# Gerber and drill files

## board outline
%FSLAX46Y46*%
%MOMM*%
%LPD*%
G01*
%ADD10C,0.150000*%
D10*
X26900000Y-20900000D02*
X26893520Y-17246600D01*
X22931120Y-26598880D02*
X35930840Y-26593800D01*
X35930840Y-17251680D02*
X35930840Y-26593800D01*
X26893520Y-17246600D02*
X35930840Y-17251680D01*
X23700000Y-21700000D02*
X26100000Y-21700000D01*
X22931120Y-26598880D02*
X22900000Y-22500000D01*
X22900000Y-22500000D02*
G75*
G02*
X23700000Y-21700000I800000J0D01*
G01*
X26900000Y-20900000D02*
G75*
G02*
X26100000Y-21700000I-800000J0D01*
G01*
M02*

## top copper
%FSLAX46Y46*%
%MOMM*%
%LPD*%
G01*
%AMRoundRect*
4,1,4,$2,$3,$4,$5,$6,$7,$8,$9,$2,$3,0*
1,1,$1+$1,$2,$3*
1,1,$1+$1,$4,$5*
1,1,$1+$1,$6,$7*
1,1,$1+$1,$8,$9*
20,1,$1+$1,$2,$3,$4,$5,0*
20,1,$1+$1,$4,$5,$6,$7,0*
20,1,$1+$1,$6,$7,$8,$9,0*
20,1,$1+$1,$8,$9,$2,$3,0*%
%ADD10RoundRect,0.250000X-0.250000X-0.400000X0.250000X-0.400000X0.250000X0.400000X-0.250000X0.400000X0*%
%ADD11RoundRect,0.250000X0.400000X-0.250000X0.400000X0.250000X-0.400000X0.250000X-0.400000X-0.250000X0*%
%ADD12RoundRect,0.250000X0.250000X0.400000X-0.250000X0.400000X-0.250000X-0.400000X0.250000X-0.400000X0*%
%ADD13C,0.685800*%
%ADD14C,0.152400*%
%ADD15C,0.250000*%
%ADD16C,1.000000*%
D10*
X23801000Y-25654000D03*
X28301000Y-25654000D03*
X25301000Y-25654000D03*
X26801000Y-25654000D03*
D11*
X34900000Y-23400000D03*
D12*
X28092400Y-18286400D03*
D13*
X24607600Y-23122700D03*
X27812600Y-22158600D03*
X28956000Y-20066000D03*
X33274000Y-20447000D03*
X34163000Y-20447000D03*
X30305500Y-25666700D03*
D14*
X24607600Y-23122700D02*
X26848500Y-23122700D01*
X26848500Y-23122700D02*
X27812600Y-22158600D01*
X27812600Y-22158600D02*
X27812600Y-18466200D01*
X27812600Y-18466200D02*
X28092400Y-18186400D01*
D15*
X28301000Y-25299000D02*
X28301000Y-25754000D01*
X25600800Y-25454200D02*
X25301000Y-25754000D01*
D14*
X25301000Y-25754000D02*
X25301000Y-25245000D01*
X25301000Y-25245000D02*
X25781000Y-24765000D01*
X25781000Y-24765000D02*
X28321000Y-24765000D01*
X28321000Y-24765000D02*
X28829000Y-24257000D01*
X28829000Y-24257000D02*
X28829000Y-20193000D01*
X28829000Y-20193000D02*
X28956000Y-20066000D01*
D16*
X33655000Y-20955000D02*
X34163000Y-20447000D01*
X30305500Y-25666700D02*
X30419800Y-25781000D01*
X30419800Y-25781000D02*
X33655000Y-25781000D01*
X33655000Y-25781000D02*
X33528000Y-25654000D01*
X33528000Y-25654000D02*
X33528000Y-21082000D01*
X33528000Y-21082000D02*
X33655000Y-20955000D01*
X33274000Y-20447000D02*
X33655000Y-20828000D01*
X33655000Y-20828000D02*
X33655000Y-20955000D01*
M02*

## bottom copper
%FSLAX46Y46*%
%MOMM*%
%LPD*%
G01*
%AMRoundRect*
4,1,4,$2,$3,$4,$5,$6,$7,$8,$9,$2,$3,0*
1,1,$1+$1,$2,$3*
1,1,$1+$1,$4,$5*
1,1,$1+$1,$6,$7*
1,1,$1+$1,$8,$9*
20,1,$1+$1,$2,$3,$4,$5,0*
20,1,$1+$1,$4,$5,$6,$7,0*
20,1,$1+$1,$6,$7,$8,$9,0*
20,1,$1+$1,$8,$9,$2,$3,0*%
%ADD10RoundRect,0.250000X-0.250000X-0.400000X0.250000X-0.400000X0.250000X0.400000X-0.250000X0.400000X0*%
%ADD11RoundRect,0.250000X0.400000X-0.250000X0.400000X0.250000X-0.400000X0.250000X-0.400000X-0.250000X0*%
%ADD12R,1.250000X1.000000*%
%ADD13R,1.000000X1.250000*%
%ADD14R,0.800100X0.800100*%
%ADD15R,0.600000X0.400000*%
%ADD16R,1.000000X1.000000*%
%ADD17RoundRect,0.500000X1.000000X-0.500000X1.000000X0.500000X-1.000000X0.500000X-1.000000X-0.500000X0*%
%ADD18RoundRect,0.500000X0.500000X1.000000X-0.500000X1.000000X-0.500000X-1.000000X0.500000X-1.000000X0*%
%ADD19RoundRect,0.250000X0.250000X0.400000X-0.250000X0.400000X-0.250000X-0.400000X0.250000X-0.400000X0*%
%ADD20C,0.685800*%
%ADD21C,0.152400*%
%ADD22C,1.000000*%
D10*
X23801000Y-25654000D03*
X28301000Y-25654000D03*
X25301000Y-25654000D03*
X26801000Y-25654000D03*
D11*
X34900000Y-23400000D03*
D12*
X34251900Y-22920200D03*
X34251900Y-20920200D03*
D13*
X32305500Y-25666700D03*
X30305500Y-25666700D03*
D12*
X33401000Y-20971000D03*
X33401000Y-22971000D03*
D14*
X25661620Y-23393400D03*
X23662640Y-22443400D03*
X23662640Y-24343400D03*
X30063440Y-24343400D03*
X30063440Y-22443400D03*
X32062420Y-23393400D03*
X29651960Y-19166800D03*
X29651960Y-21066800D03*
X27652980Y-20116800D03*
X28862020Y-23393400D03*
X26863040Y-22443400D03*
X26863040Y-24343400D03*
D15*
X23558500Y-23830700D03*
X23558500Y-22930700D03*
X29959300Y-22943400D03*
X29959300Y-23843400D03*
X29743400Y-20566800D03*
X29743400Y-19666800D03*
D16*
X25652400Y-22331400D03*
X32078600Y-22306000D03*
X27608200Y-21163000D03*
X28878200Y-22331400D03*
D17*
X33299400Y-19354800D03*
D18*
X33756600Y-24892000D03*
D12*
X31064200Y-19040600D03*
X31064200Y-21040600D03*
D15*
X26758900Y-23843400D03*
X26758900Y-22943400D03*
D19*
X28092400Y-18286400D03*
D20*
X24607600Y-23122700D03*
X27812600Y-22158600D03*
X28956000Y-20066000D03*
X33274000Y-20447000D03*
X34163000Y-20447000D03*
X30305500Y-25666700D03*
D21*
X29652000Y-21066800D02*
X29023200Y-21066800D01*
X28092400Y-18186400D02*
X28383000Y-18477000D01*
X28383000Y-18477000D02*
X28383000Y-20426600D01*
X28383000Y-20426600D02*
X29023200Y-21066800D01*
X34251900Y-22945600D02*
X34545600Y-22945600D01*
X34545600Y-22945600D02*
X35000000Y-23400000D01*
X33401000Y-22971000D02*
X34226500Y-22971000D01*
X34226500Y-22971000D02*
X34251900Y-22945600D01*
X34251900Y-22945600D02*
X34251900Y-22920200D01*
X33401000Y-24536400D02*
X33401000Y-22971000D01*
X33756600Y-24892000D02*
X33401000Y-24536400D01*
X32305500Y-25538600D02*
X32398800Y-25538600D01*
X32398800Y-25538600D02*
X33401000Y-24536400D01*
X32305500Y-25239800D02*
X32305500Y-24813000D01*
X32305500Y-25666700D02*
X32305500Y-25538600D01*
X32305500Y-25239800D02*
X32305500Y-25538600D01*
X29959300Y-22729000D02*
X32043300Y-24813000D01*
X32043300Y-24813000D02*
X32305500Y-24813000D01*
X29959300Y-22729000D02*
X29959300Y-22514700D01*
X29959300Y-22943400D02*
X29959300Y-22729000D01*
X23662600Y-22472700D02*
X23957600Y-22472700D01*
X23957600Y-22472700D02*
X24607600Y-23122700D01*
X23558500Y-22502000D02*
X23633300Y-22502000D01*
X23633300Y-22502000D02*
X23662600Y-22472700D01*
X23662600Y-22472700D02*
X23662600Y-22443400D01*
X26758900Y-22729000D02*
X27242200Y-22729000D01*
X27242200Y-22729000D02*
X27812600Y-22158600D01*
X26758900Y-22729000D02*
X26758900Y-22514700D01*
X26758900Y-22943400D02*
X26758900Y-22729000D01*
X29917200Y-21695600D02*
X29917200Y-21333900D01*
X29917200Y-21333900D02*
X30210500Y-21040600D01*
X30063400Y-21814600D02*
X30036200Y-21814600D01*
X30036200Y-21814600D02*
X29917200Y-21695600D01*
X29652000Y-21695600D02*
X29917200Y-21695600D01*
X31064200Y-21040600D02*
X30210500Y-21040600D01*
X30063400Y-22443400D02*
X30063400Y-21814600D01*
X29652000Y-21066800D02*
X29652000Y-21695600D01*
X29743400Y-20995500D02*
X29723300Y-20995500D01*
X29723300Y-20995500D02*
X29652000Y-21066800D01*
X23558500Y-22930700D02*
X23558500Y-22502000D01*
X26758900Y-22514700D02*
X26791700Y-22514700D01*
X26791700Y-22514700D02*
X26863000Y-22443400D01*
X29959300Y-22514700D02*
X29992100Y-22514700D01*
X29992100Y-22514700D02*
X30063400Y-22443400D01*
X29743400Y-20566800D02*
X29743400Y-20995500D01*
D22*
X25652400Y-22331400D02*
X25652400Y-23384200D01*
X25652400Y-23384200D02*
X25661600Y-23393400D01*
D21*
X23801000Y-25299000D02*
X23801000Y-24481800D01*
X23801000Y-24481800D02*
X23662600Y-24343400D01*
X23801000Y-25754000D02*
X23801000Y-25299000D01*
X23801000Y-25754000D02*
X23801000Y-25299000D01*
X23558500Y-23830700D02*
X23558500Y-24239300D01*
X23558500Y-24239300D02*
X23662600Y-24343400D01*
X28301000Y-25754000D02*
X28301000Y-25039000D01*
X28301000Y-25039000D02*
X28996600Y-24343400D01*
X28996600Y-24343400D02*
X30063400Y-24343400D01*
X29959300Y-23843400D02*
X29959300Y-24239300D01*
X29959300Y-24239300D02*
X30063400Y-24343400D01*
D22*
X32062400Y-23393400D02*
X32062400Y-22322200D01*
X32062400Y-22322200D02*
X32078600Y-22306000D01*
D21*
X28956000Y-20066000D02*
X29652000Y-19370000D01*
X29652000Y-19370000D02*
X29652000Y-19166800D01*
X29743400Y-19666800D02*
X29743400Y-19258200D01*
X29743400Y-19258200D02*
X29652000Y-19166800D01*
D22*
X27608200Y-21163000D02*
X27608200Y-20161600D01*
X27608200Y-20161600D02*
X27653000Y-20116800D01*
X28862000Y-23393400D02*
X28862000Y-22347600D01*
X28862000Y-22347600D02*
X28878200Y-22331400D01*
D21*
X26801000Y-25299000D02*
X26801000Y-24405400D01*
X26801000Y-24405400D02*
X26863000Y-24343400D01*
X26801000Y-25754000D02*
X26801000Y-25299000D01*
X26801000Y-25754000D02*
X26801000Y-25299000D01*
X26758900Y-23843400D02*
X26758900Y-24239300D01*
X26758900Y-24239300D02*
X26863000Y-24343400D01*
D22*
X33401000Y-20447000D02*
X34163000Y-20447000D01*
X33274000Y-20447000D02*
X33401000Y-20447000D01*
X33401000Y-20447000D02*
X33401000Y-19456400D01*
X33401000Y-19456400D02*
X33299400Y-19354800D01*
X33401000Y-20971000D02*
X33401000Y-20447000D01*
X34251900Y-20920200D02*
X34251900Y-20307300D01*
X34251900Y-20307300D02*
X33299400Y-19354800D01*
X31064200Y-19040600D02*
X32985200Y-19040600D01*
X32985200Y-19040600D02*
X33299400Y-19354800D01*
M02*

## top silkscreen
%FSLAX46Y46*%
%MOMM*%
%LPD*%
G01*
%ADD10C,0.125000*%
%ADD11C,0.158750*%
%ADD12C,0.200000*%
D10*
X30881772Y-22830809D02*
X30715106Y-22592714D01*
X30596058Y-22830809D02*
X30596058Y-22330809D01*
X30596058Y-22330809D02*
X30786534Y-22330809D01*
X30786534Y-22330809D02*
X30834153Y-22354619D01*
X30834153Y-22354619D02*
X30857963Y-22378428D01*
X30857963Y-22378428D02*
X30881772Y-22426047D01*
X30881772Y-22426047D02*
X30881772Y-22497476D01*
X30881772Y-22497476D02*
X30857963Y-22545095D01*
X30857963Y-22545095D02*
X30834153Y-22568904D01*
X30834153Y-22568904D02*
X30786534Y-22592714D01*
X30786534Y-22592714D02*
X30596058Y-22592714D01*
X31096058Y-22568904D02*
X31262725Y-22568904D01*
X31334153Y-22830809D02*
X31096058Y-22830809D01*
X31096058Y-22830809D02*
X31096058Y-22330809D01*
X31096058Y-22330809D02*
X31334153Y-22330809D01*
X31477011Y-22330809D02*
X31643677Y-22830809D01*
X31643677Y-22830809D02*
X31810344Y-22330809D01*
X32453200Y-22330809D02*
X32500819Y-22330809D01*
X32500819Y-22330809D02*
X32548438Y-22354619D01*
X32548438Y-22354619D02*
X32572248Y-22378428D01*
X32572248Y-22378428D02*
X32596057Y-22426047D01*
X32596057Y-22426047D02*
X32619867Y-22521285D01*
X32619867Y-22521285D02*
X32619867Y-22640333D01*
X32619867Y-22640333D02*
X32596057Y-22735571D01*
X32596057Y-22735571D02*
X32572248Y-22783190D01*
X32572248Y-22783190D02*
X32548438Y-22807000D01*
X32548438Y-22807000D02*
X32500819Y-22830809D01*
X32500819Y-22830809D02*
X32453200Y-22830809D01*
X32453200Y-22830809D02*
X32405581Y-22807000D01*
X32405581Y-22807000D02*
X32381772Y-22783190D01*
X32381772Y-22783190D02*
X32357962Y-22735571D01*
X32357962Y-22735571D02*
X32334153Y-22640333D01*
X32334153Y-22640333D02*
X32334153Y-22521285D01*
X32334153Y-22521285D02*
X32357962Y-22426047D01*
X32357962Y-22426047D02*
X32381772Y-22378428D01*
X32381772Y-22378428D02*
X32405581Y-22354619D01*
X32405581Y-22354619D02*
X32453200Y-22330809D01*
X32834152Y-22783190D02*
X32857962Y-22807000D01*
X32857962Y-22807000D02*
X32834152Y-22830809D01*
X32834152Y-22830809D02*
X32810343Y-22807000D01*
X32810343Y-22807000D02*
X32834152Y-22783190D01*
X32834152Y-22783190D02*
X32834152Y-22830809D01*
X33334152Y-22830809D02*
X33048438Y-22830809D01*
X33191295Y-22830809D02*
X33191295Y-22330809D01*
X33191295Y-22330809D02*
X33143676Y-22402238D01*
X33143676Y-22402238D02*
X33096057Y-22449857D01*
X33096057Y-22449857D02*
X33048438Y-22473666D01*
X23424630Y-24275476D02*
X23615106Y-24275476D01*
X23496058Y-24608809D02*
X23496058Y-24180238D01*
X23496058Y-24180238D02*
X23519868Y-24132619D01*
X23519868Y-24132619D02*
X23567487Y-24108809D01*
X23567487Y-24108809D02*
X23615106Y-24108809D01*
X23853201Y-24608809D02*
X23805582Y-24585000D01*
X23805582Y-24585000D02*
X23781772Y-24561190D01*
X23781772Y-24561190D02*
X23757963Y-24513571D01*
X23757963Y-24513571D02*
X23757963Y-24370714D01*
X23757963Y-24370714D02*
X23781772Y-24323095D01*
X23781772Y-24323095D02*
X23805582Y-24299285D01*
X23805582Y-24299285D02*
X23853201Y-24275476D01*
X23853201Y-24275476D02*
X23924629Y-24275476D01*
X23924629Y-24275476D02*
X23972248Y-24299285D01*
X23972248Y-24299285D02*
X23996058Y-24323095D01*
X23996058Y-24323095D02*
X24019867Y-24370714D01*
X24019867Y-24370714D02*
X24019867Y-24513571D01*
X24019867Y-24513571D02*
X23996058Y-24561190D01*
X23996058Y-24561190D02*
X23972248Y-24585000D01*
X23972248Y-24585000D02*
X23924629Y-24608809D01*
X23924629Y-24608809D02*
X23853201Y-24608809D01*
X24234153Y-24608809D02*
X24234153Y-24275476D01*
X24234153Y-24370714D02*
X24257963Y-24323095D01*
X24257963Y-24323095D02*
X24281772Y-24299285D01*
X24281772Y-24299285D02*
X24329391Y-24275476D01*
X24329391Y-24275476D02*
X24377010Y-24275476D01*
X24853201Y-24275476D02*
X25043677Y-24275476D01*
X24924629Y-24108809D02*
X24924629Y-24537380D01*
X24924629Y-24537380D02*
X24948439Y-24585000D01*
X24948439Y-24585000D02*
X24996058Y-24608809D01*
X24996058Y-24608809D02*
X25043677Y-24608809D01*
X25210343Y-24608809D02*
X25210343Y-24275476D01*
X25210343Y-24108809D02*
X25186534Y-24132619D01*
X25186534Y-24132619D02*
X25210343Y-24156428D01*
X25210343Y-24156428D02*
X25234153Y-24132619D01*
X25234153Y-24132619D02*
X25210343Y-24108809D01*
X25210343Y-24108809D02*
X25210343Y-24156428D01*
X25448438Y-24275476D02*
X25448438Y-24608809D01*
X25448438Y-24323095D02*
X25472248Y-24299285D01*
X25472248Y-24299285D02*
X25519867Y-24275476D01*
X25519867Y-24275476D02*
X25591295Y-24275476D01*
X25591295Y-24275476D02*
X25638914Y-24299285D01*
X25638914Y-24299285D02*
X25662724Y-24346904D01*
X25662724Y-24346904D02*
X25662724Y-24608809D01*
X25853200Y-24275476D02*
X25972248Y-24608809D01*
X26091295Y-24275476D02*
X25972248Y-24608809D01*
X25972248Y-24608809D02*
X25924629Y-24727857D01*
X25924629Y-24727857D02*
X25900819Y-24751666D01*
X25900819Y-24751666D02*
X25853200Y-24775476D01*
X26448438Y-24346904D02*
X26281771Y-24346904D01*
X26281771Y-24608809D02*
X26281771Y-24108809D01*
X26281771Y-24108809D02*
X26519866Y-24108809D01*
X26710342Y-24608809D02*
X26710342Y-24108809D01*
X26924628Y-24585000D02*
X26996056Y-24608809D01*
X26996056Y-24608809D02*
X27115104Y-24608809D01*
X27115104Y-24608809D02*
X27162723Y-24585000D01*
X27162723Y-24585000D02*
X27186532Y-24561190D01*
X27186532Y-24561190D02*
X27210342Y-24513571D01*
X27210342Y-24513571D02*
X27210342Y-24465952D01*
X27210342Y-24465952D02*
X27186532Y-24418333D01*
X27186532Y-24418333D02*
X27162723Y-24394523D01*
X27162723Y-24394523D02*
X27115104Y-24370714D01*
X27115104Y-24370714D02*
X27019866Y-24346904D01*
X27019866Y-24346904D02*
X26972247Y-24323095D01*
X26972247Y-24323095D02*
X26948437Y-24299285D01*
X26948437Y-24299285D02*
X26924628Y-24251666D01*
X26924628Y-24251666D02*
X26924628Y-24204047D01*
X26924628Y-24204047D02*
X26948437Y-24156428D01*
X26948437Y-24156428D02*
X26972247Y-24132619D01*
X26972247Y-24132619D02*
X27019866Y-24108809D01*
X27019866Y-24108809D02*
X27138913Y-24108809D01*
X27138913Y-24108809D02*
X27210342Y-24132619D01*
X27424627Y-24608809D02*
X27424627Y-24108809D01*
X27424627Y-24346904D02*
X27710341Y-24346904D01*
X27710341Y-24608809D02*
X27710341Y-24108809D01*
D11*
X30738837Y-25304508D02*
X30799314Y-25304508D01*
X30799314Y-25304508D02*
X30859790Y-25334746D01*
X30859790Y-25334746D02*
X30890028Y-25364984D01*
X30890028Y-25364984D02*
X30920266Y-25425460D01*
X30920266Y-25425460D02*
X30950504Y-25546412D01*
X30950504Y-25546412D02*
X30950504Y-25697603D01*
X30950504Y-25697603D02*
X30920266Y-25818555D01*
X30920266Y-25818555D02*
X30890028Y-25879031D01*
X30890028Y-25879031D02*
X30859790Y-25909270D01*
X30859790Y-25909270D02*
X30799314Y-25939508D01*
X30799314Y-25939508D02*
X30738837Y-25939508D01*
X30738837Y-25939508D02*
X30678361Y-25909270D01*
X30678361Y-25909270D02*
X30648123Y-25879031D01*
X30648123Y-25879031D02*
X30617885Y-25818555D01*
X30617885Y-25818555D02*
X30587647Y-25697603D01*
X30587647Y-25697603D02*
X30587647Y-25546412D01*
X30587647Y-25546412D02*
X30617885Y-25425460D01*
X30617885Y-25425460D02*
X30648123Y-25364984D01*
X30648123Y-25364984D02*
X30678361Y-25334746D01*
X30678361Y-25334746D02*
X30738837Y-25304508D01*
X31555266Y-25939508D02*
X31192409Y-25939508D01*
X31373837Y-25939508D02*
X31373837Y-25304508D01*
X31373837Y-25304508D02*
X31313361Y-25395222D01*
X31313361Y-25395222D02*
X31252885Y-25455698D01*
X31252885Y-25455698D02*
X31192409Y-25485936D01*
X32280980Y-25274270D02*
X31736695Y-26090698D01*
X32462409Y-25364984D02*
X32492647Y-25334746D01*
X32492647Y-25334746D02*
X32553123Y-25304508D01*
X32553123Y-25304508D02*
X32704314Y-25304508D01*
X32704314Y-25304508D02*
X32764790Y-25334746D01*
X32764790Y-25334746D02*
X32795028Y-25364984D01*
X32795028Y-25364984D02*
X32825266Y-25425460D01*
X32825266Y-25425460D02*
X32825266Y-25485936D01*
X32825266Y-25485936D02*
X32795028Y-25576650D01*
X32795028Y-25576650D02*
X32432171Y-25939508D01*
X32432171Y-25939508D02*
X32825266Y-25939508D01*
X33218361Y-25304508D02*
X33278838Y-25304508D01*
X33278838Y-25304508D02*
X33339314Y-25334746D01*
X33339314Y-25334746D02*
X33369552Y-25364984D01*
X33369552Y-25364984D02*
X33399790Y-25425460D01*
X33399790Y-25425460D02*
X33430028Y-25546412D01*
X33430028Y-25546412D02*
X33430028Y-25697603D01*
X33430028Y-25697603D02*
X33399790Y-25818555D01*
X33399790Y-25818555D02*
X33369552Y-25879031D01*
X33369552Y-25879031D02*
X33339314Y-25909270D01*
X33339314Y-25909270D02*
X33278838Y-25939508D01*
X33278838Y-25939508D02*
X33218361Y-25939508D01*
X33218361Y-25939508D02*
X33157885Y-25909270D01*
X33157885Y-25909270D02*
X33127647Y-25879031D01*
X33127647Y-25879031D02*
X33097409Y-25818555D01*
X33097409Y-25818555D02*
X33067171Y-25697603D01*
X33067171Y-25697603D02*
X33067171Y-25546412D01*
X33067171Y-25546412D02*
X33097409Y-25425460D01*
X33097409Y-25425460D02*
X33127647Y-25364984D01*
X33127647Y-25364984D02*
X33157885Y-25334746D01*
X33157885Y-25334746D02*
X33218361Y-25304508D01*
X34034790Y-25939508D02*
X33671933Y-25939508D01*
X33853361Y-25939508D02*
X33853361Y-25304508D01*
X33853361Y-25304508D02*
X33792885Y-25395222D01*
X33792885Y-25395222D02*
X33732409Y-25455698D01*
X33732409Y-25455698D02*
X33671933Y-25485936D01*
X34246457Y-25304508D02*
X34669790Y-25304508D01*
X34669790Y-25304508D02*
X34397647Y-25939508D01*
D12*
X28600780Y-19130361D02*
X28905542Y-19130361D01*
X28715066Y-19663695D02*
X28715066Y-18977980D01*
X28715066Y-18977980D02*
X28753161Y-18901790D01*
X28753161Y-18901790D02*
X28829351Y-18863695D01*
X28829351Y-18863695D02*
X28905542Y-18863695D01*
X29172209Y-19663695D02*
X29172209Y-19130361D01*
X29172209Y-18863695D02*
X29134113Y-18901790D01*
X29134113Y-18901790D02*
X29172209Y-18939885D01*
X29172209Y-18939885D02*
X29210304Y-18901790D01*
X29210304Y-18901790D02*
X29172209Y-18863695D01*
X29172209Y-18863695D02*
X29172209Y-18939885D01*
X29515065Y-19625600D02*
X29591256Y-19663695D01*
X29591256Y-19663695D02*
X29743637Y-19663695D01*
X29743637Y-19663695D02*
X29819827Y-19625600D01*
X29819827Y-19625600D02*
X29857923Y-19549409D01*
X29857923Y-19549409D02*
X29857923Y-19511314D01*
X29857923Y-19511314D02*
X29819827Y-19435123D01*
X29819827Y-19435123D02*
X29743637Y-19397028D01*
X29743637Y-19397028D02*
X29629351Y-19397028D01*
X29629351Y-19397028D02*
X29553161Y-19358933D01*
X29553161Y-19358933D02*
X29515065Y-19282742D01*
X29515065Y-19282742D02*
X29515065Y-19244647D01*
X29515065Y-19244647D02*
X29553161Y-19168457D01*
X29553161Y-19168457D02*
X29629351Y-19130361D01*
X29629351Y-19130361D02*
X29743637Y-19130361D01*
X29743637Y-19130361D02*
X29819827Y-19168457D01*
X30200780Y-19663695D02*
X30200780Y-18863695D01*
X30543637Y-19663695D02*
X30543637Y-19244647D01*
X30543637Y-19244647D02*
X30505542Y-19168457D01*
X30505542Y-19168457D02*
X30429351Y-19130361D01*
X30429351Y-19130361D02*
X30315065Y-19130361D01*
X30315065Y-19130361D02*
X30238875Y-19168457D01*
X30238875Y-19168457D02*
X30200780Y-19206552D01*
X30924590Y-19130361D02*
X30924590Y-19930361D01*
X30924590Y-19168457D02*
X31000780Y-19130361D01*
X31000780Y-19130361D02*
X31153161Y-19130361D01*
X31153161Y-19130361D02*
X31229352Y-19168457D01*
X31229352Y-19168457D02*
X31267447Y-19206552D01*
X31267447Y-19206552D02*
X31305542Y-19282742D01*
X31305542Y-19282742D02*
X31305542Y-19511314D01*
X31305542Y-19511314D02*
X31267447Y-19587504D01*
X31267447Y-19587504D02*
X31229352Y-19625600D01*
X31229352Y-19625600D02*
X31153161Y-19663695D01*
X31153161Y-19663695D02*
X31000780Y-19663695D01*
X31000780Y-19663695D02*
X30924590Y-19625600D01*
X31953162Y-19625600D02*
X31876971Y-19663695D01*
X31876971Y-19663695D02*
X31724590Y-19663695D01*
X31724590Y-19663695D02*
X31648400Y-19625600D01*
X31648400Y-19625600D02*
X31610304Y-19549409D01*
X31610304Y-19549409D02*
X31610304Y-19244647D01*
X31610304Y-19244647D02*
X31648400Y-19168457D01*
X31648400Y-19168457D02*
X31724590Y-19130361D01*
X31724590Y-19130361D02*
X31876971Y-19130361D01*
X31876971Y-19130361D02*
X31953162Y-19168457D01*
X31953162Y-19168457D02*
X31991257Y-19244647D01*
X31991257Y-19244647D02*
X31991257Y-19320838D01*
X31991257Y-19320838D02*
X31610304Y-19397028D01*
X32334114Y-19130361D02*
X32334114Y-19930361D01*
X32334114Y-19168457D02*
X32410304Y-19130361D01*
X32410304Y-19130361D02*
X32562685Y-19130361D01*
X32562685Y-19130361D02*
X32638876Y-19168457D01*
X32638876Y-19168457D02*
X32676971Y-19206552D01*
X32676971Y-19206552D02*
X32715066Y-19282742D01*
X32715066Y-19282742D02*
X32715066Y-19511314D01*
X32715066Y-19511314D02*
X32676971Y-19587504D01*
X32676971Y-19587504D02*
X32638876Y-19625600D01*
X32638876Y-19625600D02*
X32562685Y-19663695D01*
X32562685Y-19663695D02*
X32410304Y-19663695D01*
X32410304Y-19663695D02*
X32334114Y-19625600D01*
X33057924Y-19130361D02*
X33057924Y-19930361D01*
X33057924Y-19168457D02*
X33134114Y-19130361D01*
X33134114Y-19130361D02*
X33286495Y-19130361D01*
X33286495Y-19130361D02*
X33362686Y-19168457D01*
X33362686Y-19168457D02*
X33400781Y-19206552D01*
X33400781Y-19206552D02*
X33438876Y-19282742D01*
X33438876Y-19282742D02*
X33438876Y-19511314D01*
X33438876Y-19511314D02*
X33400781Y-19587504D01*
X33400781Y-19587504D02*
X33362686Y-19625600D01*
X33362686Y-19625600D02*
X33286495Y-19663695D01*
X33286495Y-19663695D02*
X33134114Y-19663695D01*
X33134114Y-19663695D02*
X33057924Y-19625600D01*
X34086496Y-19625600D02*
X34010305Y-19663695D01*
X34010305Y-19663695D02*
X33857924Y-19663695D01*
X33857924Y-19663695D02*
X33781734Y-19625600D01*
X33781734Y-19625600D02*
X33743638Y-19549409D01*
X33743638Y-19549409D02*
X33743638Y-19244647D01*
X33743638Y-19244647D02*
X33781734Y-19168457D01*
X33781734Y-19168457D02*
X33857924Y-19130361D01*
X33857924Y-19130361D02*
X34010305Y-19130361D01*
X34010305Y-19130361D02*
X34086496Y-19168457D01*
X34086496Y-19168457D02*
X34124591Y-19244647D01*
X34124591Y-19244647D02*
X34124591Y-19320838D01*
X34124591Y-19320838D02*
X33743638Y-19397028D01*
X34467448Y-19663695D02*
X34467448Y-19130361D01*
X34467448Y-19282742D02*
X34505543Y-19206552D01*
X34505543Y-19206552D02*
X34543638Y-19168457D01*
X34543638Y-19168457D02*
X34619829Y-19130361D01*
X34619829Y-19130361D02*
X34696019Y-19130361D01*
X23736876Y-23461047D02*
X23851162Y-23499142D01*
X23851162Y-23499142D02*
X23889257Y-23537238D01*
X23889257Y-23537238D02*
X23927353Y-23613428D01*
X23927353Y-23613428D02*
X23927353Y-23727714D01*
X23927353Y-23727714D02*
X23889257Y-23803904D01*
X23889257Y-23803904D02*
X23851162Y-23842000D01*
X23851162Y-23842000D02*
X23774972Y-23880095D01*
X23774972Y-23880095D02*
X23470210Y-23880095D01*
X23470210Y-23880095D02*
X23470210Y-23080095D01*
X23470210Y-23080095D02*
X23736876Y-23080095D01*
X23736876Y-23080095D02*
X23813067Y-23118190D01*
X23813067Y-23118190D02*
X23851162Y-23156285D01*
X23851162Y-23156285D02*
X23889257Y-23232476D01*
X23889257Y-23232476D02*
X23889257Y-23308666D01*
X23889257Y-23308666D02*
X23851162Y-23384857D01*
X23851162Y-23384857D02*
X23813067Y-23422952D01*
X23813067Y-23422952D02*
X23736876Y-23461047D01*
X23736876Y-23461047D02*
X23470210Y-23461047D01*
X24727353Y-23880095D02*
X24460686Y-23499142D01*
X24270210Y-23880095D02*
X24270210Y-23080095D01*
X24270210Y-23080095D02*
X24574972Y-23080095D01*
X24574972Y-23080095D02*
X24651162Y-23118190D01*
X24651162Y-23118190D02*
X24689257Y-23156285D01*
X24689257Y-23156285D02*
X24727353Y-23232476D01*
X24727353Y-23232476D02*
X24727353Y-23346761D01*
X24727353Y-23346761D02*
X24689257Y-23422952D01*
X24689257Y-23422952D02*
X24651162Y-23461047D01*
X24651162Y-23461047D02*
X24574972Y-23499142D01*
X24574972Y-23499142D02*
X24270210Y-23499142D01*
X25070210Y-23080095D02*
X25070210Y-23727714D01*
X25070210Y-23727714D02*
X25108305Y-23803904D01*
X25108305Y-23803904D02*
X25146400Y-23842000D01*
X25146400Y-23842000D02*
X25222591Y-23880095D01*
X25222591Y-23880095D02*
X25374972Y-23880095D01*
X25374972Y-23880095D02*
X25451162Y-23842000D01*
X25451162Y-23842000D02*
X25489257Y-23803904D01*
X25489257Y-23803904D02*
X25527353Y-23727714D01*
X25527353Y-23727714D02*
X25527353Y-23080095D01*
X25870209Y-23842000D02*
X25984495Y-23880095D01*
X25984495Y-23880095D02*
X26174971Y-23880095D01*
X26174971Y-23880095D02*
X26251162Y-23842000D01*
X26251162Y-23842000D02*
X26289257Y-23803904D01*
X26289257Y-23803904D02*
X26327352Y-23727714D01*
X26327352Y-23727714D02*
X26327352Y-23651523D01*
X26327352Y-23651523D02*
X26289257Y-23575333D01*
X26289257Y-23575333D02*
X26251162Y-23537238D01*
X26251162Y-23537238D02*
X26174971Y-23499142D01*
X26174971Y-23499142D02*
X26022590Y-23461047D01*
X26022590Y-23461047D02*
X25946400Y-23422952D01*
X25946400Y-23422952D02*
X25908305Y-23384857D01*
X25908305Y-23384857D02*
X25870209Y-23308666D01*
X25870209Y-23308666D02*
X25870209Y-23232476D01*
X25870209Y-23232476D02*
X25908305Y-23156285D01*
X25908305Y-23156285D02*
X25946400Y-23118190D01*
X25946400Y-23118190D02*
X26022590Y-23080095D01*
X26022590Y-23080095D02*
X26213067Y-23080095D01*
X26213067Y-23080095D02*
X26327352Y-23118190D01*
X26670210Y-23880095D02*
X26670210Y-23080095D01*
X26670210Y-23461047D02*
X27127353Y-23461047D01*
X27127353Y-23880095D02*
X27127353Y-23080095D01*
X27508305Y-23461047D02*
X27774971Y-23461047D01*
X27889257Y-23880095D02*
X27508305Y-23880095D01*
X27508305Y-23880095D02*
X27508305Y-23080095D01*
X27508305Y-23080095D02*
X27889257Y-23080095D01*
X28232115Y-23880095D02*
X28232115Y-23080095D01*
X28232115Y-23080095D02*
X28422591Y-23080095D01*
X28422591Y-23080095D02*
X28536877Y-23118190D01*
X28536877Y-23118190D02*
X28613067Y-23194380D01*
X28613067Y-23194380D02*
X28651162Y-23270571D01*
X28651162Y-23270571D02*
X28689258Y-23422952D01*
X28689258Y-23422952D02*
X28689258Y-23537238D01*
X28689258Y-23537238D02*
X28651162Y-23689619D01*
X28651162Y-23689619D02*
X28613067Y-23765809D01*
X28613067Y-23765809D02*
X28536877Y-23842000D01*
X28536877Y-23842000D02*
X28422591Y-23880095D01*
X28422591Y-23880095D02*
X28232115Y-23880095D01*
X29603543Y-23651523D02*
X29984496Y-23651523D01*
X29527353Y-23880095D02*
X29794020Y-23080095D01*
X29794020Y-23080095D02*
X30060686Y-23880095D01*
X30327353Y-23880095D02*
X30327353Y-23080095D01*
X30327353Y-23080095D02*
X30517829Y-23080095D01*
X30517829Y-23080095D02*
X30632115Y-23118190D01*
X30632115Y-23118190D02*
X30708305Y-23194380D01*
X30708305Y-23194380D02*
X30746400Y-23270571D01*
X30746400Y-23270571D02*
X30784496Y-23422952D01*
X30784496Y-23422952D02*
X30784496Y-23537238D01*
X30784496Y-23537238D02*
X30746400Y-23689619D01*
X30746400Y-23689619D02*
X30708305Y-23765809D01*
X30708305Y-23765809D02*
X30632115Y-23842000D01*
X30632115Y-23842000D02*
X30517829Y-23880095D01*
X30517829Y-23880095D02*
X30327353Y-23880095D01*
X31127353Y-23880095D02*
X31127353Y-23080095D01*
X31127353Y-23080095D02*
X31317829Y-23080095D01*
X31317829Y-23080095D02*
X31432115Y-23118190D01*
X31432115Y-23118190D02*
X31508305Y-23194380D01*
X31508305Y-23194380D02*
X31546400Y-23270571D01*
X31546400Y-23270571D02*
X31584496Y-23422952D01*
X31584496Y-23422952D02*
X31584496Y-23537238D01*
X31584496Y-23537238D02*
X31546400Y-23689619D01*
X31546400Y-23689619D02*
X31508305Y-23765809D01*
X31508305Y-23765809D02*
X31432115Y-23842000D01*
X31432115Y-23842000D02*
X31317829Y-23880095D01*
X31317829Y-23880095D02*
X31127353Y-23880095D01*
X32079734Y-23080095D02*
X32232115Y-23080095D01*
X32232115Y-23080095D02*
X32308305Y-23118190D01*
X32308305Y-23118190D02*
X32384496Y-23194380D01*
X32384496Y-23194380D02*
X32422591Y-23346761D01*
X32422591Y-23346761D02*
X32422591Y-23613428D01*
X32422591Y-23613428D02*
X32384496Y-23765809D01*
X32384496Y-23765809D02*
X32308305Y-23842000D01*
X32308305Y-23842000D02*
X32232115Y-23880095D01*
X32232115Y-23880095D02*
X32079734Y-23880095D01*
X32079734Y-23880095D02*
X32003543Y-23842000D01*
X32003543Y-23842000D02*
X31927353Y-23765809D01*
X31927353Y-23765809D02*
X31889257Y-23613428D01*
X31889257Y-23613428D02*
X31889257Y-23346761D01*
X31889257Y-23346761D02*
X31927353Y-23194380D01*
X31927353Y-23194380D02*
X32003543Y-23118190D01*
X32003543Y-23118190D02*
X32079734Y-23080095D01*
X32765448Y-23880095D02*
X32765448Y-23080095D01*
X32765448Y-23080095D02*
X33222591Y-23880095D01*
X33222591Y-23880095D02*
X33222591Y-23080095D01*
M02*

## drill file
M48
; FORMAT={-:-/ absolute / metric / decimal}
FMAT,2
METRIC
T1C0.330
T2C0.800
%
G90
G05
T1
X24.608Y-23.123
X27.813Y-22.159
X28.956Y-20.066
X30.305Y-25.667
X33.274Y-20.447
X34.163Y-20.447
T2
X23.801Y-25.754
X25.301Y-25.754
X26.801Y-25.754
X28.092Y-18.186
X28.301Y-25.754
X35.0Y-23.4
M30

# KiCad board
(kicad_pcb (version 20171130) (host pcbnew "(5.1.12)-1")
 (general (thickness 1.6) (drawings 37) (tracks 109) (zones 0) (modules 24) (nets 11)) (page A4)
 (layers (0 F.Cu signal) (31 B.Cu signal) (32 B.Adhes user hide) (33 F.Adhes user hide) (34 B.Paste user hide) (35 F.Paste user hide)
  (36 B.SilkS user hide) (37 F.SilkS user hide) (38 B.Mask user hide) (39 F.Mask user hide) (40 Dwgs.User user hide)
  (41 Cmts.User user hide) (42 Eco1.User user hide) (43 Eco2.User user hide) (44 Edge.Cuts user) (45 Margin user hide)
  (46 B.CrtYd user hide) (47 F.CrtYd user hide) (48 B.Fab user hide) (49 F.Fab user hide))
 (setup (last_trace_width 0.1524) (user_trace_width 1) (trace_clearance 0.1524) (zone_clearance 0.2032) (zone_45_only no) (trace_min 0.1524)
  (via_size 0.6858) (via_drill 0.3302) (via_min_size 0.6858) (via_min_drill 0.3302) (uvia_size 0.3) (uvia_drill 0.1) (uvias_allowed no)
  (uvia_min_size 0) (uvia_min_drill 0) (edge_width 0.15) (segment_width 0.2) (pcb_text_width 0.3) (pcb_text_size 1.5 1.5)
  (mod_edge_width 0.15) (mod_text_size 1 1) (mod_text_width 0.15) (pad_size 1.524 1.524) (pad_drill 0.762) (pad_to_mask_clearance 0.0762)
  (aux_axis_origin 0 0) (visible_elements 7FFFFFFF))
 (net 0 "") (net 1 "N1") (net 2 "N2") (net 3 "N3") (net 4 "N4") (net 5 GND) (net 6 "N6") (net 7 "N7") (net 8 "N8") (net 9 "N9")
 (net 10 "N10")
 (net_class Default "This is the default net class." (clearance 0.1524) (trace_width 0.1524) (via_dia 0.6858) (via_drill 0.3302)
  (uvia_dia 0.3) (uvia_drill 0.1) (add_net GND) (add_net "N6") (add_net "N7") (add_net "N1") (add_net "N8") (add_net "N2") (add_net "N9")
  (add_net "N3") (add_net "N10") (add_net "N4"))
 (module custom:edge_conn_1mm (layer F.Cu) (at 23.801 25.754)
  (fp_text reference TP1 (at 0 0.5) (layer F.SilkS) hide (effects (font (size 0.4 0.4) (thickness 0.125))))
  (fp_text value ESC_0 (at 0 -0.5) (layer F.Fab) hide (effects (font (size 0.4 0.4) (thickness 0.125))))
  (pad 1 thru_hole roundrect (at 0 0) (size 1 1.3) (drill 0.8 (offset 0 -0.1)) (layers *.Cu *.Mask) (roundrect_rratio 0.25) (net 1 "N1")))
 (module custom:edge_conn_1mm (layer F.Cu) (at 28.301 25.754)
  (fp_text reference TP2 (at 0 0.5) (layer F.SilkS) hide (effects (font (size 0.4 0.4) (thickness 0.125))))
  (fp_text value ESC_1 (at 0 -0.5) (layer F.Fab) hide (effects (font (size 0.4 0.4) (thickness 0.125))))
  (pad 1 thru_hole roundrect (at 0 0) (size 1 1.3) (drill 0.8 (offset 0 -0.1)) (layers *.Cu *.Mask) (roundrect_rratio 0.25) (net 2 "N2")))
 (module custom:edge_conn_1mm (layer F.Cu) (at 25.301 25.754)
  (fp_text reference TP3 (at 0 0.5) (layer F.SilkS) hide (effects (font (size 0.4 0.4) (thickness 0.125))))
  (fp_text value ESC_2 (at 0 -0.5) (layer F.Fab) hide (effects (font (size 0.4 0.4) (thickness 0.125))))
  (pad 1 thru_hole roundrect (at 0 0) (size 1 1.3) (drill 0.8 (offset 0 -0.1)) (layers *.Cu *.Mask) (roundrect_rratio 0.25) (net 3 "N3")))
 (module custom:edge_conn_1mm (layer F.Cu) (at 26.801 25.754)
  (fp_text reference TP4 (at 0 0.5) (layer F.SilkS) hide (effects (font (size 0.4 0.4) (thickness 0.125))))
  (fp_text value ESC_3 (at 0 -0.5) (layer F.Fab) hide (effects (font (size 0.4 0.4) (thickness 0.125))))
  (pad 1 thru_hole roundrect (at 0 0) (size 1 1.3) (drill 0.8 (offset 0 -0.1)) (layers *.Cu *.Mask) (roundrect_rratio 0.25) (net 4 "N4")))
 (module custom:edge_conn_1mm (layer F.Cu) (at 35 23.4 90)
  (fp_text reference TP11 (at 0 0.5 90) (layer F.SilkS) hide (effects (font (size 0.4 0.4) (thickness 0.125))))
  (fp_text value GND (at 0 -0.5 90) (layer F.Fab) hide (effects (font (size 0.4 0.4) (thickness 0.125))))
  (pad 1 thru_hole roundrect (at 0 0 90) (size 1 1.3) (drill 0.8 (offset 0 -0.1)) (layers *.Cu *.Mask) (roundrect_rratio 0.25) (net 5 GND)))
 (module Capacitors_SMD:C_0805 (layer B.Cu) (at 34.2519 21.9202 270)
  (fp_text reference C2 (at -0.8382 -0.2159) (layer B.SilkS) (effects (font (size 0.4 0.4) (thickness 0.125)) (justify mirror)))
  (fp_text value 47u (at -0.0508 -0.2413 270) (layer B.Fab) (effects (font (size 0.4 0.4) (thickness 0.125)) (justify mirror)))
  (pad 2 smd rect (at 1 0 270) (size 1 1.25) (layers B.Cu B.Paste B.Mask) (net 5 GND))
  (pad 1 smd rect (at -1 0 270) (size 1 1.25) (layers B.Cu B.Paste B.Mask) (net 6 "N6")))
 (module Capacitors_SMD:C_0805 (layer B.Cu) (at 31.3055 25.6667)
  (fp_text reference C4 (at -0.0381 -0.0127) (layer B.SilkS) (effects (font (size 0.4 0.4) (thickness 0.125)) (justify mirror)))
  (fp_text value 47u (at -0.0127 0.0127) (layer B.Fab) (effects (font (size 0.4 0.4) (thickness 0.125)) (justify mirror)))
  (pad 2 smd rect (at 1 0) (size 1 1.25) (layers B.Cu B.Paste B.Mask) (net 5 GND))
  (pad 1 smd rect (at -1 0) (size 1 1.25) (layers B.Cu B.Paste B.Mask) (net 6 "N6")))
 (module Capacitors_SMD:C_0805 (layer B.Cu) (at 33.401 21.971 270)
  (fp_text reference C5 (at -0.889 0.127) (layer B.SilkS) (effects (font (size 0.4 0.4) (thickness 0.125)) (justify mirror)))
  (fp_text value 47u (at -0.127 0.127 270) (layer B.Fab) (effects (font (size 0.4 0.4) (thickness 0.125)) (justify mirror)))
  (pad 1 smd rect (at -1 0 270) (size 1 1.25) (layers B.Cu B.Paste B.Mask) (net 6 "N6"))
  (pad 2 smd rect (at 1 0 270) (size 1 1.25) (layers B.Cu B.Paste B.Mask) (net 5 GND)))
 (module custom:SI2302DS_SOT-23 (layer B.Cu) (at 24.6634 23.3934 90)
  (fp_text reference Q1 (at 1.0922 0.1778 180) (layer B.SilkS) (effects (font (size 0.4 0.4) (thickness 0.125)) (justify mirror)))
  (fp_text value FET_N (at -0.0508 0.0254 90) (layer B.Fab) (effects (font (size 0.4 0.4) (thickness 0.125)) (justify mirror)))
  (pad D smd rect (at 0 0.99822 90) (size 0.8001 0.8001) (layers B.Cu B.Paste B.Mask) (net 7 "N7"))
  (pad S smd rect (at 0.95 -1.00076 90) (size 0.8001 0.8001) (layers B.Cu B.Paste B.Mask) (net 5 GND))
  (pad G smd rect (at -0.95 -1.00076 90) (size 0.8001 0.8001) (layers B.Cu B.Paste B.Mask) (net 1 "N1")))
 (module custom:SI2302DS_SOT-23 (layer B.Cu) (at 31.0642 23.3934 90)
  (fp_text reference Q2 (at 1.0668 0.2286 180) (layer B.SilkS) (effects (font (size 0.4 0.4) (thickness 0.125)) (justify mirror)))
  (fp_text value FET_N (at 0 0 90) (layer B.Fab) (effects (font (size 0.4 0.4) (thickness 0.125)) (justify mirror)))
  (pad G smd rect (at -0.95 -1.00076 90) (size 0.8001 0.8001) (layers B.Cu B.Paste B.Mask) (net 2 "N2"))
  (pad S smd rect (at 0.95 -1.00076 90) (size 0.8001 0.8001) (layers B.Cu B.Paste B.Mask) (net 5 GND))
  (pad D smd rect (at 0 0.99822 90) (size 0.8001 0.8001) (layers B.Cu B.Paste B.Mask) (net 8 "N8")))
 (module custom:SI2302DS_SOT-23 (layer B.Cu) (at 28.6512 20.1168 270)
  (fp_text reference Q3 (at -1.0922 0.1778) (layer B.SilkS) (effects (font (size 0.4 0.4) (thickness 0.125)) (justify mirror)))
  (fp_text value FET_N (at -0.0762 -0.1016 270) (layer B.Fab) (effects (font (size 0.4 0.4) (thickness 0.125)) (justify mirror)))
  (pad G smd rect (at -0.95 -1.00076 270) (size 0.8001 0.8001) (layers B.Cu B.Paste B.Mask) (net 3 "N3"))
  (pad S smd rect (at 0.95 -1.00076 270) (size 0.8001 0.8001) (layers B.Cu B.Paste B.Mask) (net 5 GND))
  (pad D smd rect (at 0 0.99822 270) (size 0.8001 0.8001) (layers B.Cu B.Paste B.Mask) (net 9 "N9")))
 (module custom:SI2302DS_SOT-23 (layer B.Cu) (at 27.8638 23.3934 90)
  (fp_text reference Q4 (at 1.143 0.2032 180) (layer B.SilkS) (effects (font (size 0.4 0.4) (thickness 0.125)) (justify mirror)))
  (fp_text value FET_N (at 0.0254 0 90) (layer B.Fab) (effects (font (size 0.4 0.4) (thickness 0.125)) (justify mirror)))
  (pad D smd rect (at 0 0.99822 90) (size 0.8001 0.8001) (layers B.Cu B.Paste B.Mask) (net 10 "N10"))
  (pad S smd rect (at 0.95 -1.00076 90) (size 0.8001 0.8001) (layers B.Cu B.Paste B.Mask) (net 5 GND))
  (pad G smd rect (at -0.95 -1.00076 90) (size 0.8001 0.8001) (layers B.Cu B.Paste B.Mask) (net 4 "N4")))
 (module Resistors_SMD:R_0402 (layer B.Cu) (at 23.5585 23.3807 90)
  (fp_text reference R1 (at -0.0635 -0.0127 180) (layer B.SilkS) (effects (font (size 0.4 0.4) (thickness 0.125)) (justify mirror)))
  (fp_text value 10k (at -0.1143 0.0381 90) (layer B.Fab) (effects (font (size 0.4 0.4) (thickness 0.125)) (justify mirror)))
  (pad 1 smd rect (at -0.45 0 90) (size 0.4 0.6) (layers B.Cu B.Paste B.Mask) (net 1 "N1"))
  (pad 2 smd rect (at 0.45 0 90) (size 0.4 0.6) (layers B.Cu B.Paste B.Mask) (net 5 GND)))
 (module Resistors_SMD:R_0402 (layer B.Cu) (at 29.9593 23.3934 90)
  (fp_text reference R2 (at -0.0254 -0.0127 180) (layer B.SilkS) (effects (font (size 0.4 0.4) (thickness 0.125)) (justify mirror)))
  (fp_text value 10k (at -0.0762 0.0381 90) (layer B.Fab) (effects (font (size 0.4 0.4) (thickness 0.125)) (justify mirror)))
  (pad 2 smd rect (at 0.45 0 90) (size 0.4 0.6) (layers B.Cu B.Paste B.Mask) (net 5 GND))
  (pad 1 smd rect (at -0.45 0 90) (size 0.4 0.6) (layers B.Cu B.Paste B.Mask) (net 2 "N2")))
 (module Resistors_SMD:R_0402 (layer B.Cu) (at 29.7434 20.1168 270)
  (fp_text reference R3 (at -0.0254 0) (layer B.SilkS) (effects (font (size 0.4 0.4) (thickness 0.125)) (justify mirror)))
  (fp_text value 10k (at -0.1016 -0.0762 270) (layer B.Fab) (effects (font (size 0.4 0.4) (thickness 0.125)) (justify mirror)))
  (pad 2 smd rect (at 0.45 0 270) (size 0.4 0.6) (layers B.Cu B.Paste B.Mask) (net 5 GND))
  (pad 1 smd rect (at -0.45 0 270) (size 0.4 0.6) (layers B.Cu B.Paste B.Mask) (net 3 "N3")))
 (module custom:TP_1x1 (layer B.Cu) (at 25.5524 22.6314)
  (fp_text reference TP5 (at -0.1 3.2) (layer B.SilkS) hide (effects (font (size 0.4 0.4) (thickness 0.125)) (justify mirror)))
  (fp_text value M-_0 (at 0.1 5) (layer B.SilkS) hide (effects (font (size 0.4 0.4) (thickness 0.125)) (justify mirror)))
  (pad 1 smd rect (at 0.1 -0.3) (size 1 1) (layers B.Cu B.Mask) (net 7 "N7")))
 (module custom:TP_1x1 (layer B.Cu) (at 31.9786 22.606)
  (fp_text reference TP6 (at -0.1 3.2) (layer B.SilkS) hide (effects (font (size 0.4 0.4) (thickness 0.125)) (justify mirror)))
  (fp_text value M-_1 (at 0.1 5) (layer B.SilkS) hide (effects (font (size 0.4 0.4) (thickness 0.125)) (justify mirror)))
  (pad 1 smd rect (at 0.1 -0.3) (size 1 1) (layers B.Cu B.Mask) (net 8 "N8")))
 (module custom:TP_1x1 (layer B.Cu) (at 27.5082 21.463)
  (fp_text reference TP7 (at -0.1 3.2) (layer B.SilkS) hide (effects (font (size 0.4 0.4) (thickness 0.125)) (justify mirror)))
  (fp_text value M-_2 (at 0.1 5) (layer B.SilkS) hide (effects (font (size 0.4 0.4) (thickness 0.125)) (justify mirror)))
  (pad 1 smd rect (at 0.1 -0.3) (size 1 1) (layers B.Cu B.Mask) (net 9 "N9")))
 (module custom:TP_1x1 (layer B.Cu) (at 28.7782 22.6314)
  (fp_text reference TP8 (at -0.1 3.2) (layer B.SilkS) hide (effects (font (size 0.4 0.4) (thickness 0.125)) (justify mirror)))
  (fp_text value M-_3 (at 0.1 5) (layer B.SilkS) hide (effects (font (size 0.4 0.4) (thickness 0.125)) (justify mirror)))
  (pad 1 smd rect (at 0.1 -0.3) (size 1 1) (layers B.Cu B.Mask) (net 10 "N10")))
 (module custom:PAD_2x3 (layer B.Cu) (at 33.2994 19.3548 90)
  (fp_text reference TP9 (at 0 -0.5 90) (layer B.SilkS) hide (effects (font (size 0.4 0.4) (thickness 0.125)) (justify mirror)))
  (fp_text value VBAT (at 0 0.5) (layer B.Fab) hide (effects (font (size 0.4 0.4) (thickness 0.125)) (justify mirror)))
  (pad 1 smd roundrect (at 0 0 90) (size 2 3) (layers B.Cu B.Mask) (roundrect_rratio 0.25) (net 6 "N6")))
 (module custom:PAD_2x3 (layer B.Cu) (at 33.7566 24.892 180)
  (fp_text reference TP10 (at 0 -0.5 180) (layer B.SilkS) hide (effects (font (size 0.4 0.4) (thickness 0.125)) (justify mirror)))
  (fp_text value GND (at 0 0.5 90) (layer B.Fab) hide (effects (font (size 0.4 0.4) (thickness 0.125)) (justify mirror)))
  (pad 1 smd roundrect (at 0 0 180) (size 2 3) (layers B.Cu B.Mask) (roundrect_rratio 0.25) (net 5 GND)))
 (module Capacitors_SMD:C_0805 (layer B.Cu) (at 31.0642 20.0406 270)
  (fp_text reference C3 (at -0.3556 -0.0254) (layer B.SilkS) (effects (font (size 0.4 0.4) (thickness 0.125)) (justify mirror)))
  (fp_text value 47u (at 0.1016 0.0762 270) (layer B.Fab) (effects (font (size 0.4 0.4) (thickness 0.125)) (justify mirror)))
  (pad 1 smd rect (at -1 0 270) (size 1 1.25) (layers B.Cu B.Paste B.Mask) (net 6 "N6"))
  (pad 2 smd rect (at 1 0 270) (size 1 1.25) (layers B.Cu B.Paste B.Mask) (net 5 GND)))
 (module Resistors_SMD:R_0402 (layer B.Cu) (at 26.7589 23.3934 90)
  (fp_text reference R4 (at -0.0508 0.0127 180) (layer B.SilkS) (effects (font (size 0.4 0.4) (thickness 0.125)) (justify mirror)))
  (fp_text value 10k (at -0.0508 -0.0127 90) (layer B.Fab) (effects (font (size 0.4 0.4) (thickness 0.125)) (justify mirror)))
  (pad 1 smd rect (at -0.45 0 90) (size 0.4 0.6) (layers B.Cu B.Paste B.Mask) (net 4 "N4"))
  (pad 2 smd rect (at 0.45 0 90) (size 0.4 0.6) (layers B.Cu B.Paste B.Mask) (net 5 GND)))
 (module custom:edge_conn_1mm (layer F.Cu) (at 28.0924 18.1864 180)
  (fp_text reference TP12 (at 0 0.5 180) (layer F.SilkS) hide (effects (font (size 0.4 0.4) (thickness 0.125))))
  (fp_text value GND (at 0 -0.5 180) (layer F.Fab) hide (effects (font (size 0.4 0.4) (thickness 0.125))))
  (pad 1 thru_hole roundrect (at 0 0 180) (size 1 1.3) (drill 0.8 (offset 0 -0.1)) (layers *.Cu *.Mask) (roundrect_rratio 0.25) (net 5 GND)))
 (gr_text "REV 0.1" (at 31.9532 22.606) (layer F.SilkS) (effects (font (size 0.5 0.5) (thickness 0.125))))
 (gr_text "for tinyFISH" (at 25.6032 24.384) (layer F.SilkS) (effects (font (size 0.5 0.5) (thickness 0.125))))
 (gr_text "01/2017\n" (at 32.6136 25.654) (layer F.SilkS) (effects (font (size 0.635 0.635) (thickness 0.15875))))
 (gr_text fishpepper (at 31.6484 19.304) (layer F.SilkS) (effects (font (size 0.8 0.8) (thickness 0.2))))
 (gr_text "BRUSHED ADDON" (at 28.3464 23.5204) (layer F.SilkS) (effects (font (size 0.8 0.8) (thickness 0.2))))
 (gr_line (start 26.9 20.9) (end 26.89352 17.2466) (angle 90) (layer Edge.Cuts) (width 0.15))
 (gr_line (start 22.93112 26.59888) (end 35.93084 26.5938) (angle 90) (layer Edge.Cuts) (width 0.15))
 (gr_line (start 35.93084 17.25168) (end 35.93084 26.5938) (angle 90) (layer Edge.Cuts) (width 0.15))
 (gr_line (start 26.89352 17.2466) (end 35.93084 17.25168) (angle 90) (layer Edge.Cuts) (width 0.15))
 (gr_line (start 23.7 21.7) (end 26.1 21.7) (angle 90) (layer Edge.Cuts) (width 0.15))
 (gr_line (start 22.93112 26.59888) (end 22.9 22.5) (angle 90) (layer Edge.Cuts) (width 0.15))
 (gr_arc (start 23.7 22.5) (end 22.9 22.5) (angle 90) (layer Edge.Cuts) (width 0.15))
 (gr_arc (start 26.1 20.9) (end 26.9 20.9) (angle 90) (layer Edge.Cuts) (width 0.15))
 (segment (start 29.652 21.0668) (end 29.0232 21.0668) (width 0.1524) (layer B.Cu) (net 5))
 (segment (start 28.0924 18.1864) (end 28.383 18.477) (width 0.1524) (layer B.Cu) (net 5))
 (segment (start 28.383 18.477) (end 28.383 20.4266) (width 0.1524) (layer B.Cu) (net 5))
 (segment (start 28.383 20.4266) (end 29.0232 21.0668) (width 0.1524) (layer B.Cu) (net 5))
 (segment (start 34.2519 22.9456) (end 34.5456 22.9456) (width 0.1524) (layer B.Cu) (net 5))
 (segment (start 34.5456 22.9456) (end 35 23.4) (width 0.1524) (layer B.Cu) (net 5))
 (segment (start 33.401 22.971) (end 34.2265 22.971) (width 0.1524) (layer B.Cu) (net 5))
 (segment (start 34.2265 22.971) (end 34.2519 22.9456) (width 0.1524) (layer B.Cu) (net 5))
 (segment (start 34.2519 22.9456) (end 34.2519 22.9202) (width 0.1524) (layer B.Cu) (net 5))
 (segment (start 33.401 24.5364) (end 33.401 22.971) (width 0.1524) (layer B.Cu) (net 5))
 (segment (start 33.7566 24.892) (end 33.401 24.5364) (width 0.1524) (layer B.Cu) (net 5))
 (segment (start 32.3055 25.5386) (end 32.3988 25.5386) (width 0.1524) (layer B.Cu) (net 5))
 (segment (start 32.3988 25.5386) (end 33.401 24.5364) (width 0.1524) (layer B.Cu) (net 5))
 (segment (start 32.3055 25.2398) (end 32.3055 24.813) (width 0.1524) (layer B.Cu) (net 5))
 (segment (start 32.3055 25.6667) (end 32.3055 25.5386) (width 0.1524) (layer B.Cu) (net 5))
 (segment (start 32.3055 25.2398) (end 32.3055 25.5386) (width 0.1524) (layer B.Cu) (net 5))
 (segment (start 29.9593 22.729) (end 32.0433 24.813) (width 0.1524) (layer B.Cu) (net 5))
 (segment (start 32.0433 24.813) (end 32.3055 24.813) (width 0.1524) (layer B.Cu) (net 5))
 (segment (start 29.9593 22.729) (end 29.9593 22.5147) (width 0.1524) (layer B.Cu) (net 5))
 (segment (start 29.9593 22.9434) (end 29.9593 22.729) (width 0.1524) (layer B.Cu) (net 5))
 (segment (start 23.6626 22.4727) (end 23.9576 22.4727) (width 0.1524) (layer B.Cu) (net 5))
 (segment (start 23.9576 22.4727) (end 24.6076 23.1227) (width 0.1524) (layer B.Cu) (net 5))
 (segment (start 23.5585 22.502) (end 23.6333 22.502) (width 0.1524) (layer B.Cu) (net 5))
 (segment (start 23.6333 22.502) (end 23.6626 22.4727) (width 0.1524) (layer B.Cu) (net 5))
 (segment (start 23.6626 22.4727) (end 23.6626 22.4434) (width 0.1524) (layer B.Cu) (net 5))
 (segment (start 24.6076 23.1227) (end 26.8485 23.1227) (width 0.1524) (layer F.Cu) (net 5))
 (segment (start 26.8485 23.1227) (end 27.8126 22.1586) (width 0.1524) (layer F.Cu) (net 5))
 (segment (start 27.8126 22.1586) (end 27.8126 18.4662) (width 0.1524) (layer F.Cu) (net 5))
 (segment (start 27.8126 18.4662) (end 28.0924 18.1864) (width 0.1524) (layer F.Cu) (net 5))
 (segment (start 26.7589 22.729) (end 27.2422 22.729) (width 0.1524) (layer B.Cu) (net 5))
 (segment (start 27.2422 22.729) (end 27.8126 22.1586) (width 0.1524) (layer B.Cu) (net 5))
 (segment (start 26.7589 22.729) (end 26.7589 22.5147) (width 0.1524) (layer B.Cu) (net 5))
 (segment (start 26.7589 22.9434) (end 26.7589 22.729) (width 0.1524) (layer B.Cu) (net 5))
 (segment (start 29.9172 21.6956) (end 29.9172 21.3339) (width 0.1524) (layer B.Cu) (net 5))
 (segment (start 29.9172 21.3339) (end 30.2105 21.0406) (width 0.1524) (layer B.Cu) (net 5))
 (segment (start 30.0634 21.8146) (end 30.0362 21.8146) (width 0.1524) (layer B.Cu) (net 5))
 (segment (start 30.0362 21.8146) (end 29.9172 21.6956) (width 0.1524) (layer B.Cu) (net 5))
 (segment (start 29.652 21.6956) (end 29.9172 21.6956) (width 0.1524) (layer B.Cu) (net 5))
 (segment (start 31.0642 21.0406) (end 30.2105 21.0406) (width 0.1524) (layer B.Cu) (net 5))
 (segment (start 30.0634 22.4434) (end 30.0634 21.8146) (width 0.1524) (layer B.Cu) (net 5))
 (segment (start 29.652 21.0668) (end 29.652 21.6956) (width 0.1524) (layer B.Cu) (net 5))
 (segment (start 29.7434 20.9955) (end 29.7233 20.9955) (width 0.1524) (layer B.Cu) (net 5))
 (segment (start 29.7233 20.9955) (end 29.652 21.0668) (width 0.1524) (layer B.Cu) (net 5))
 (segment (start 23.5585 22.9307) (end 23.5585 22.502) (width 0.1524) (layer B.Cu) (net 5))
 (segment (start 26.7589 22.5147) (end 26.7917 22.5147) (width 0.1524) (layer B.Cu) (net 5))
 (segment (start 26.7917 22.5147) (end 26.863 22.4434) (width 0.1524) (layer B.Cu) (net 5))
 (segment (start 29.9593 22.5147) (end 29.9921 22.5147) (width 0.1524) (layer B.Cu) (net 5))
 (segment (start 29.9921 22.5147) (end 30.0634 22.4434) (width 0.1524) (layer B.Cu) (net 5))
 (segment (start 29.7434 20.5668) (end 29.7434 20.9955) (width 0.1524) (layer B.Cu) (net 5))
 (via (at 24.6076 23.1227) (size 0.6858) (layers F.Cu B.Cu) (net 5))
 (via (at 27.8126 22.1586) (size 0.6858) (layers F.Cu B.Cu) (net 5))
 (segment (start 25.6524 22.3314) (end 25.6524 23.3842) (width 1) (layer B.Cu) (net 7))
 (segment (start 25.6524 23.3842) (end 25.6616 23.3934) (width 1) (layer B.Cu) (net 7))
 (segment (start 23.801 25.299) (end 23.801 24.4818) (width 0.1524) (layer B.Cu) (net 1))
 (segment (start 23.801 24.4818) (end 23.6626 24.3434) (width 0.1524) (layer B.Cu) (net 1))
 (segment (start 23.801 25.754) (end 23.801 25.299) (width 0.1524) (layer B.Cu) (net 1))
 (segment (start 23.801 25.754) (end 23.801 25.299) (width 0.1524) (layer B.Cu) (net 1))
 (segment (start 23.5585 23.8307) (end 23.5585 24.2393) (width 0.1524) (layer B.Cu) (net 1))
 (segment (start 23.5585 24.2393) (end 23.6626 24.3434) (width 0.1524) (layer B.Cu) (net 1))
 (segment (start 28.301 25.299) (end 28.301 25.754) (width 0.25) (layer F.Cu) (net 2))
 (segment (start 28.301 25.754) (end 28.301 25.039) (width 0.1524) (layer B.Cu) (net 2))
 (segment (start 28.301 25.039) (end 28.9966 24.3434) (width 0.1524) (layer B.Cu) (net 2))
 (segment (start 28.9966 24.3434) (end 30.0634 24.3434) (width 0.1524) (layer B.Cu) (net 2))
 (segment (start 29.9593 23.8434) (end 29.9593 24.2393) (width 0.1524) (layer B.Cu) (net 2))
 (segment (start 29.9593 24.2393) (end 30.0634 24.3434) (width 0.1524) (layer B.Cu) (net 2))
 (segment (start 32.0624 23.3934) (end 32.0624 22.3222) (width 1) (layer B.Cu) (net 8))
 (segment (start 32.0624 22.3222) (end 32.0786 22.306) (width 1) (layer B.Cu) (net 8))
 (segment (start 25.6008 25.4542) (end 25.301 25.754) (width 0.25) (layer F.Cu) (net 3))
 (segment (start 28.956 20.066) (end 29.652 19.37) (width 0.1524) (layer B.Cu) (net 3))
 (segment (start 29.652 19.37) (end 29.652 19.1668) (width 0.1524) (layer B.Cu) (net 3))
 (segment (start 25.301 25.754) (end 25.301 25.245) (width 0.1524) (layer F.Cu) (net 3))
 (segment (start 25.301 25.245) (end 25.781 24.765) (width 0.1524) (layer F.Cu) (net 3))
 (segment (start 25.781 24.765) (end 28.321 24.765) (width 0.1524) (layer F.Cu) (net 3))
 (segment (start 28.321 24.765) (end 28.829 24.257) (width 0.1524) (layer F.Cu) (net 3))
 (segment (start 28.829 24.257) (end 28.829 20.193) (width 0.1524) (layer F.Cu) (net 3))
 (segment (start 28.829 20.193) (end 28.956 20.066) (width 0.1524) (layer F.Cu) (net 3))
 (segment (start 29.7434 19.6668) (end 29.7434 19.2582) (width 0.1524) (layer B.Cu) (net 3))
 (segment (start 29.7434 19.2582) (end 29.652 19.1668) (width 0.1524) (layer B.Cu) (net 3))
 (via (at 28.956 20.066) (size 0.6858) (layers F.Cu B.Cu) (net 3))
 (segment (start 27.6082 21.163) (end 27.6082 20.1616) (width 1) (layer B.Cu) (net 9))
 (segment (start 27.6082 20.1616) (end 27.653 20.1168) (width 1) (layer B.Cu) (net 9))
 (segment (start 28.862 23.3934) (end 28.862 22.3476) (width 1) (layer B.Cu) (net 10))
 (segment (start 28.862 22.3476) (end 28.8782 22.3314) (width 1) (layer B.Cu) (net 10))
 (segment (start 26.801 25.299) (end 26.801 24.4054) (width 0.1524) (layer B.Cu) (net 4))
 (segment (start 26.801 24.4054) (end 26.863 24.3434) (width 0.1524) (layer B.Cu) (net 4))
 (segment (start 26.801 25.754) (end 26.801 25.299) (width 0.1524) (layer B.Cu) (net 4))
 (segment (start 26.801 25.754) (end 26.801 25.299) (width 0.1524) (layer B.Cu) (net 4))
 (segment (start 26.7589 23.8434) (end 26.7589 24.2393) (width 0.1524) (layer B.Cu) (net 4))
 (segment (start 26.7589 24.2393) (end 26.863 24.3434) (width 0.1524) (layer B.Cu) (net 4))
 (segment (start 33.401 20.447) (end 34.163 20.447) (width 1) (layer B.Cu) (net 6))
 (segment (start 33.274 20.447) (end 33.401 20.447) (width 1) (layer B.Cu) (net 6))
 (segment (start 33.401 20.447) (end 33.401 19.4564) (width 1) (layer B.Cu) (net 6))
 (segment (start 33.401 19.4564) (end 33.2994 19.3548) (width 1) (layer B.Cu) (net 6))
 (segment (start 33.401 20.971) (end 33.401 20.447) (width 1) (layer B.Cu) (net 6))
 (segment (start 33.655 20.955) (end 34.163 20.447) (width 1) (layer F.Cu) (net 6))
 (segment (start 30.3055 25.6667) (end 30.4198 25.781) (width 1) (layer F.Cu) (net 6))
 (segment (start 30.4198 25.781) (end 33.655 25.781) (width 1) (layer F.Cu) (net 6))
 (segment (start 33.655 25.781) (end 33.528 25.654) (width 1) (layer F.Cu) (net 6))
 (segment (start 33.528 25.654) (end 33.528 21.082) (width 1) (layer F.Cu) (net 6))
 (segment (start 33.528 21.082) (end 33.655 20.955) (width 1) (layer F.Cu) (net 6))
 (segment (start 33.274 20.447) (end 33.655 20.828) (width 1) (layer F.Cu) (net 6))
 (segment (start 33.655 20.828) (end 33.655 20.955) (width 1) (layer F.Cu) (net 6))
 (segment (start 34.2519 20.9202) (end 34.2519 20.3073) (width 1) (layer B.Cu) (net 6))
 (segment (start 34.2519 20.3073) (end 33.2994 19.3548) (width 1) (layer B.Cu) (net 6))
 (segment (start 31.0642 19.0406) (end 32.9852 19.0406) (width 1) (layer B.Cu) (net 6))
 (segment (start 32.9852 19.0406) (end 33.2994 19.3548) (width 1) (layer B.Cu) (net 6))
 (via (at 33.274 20.447) (size 0.6858) (layers F.Cu B.Cu) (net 6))
 (via (at 34.163 20.447) (size 0.6858) (layers F.Cu B.Cu) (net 6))
 (via (at 30.3055 25.6667) (size 0.6858) (layers F.Cu B.Cu) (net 6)))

